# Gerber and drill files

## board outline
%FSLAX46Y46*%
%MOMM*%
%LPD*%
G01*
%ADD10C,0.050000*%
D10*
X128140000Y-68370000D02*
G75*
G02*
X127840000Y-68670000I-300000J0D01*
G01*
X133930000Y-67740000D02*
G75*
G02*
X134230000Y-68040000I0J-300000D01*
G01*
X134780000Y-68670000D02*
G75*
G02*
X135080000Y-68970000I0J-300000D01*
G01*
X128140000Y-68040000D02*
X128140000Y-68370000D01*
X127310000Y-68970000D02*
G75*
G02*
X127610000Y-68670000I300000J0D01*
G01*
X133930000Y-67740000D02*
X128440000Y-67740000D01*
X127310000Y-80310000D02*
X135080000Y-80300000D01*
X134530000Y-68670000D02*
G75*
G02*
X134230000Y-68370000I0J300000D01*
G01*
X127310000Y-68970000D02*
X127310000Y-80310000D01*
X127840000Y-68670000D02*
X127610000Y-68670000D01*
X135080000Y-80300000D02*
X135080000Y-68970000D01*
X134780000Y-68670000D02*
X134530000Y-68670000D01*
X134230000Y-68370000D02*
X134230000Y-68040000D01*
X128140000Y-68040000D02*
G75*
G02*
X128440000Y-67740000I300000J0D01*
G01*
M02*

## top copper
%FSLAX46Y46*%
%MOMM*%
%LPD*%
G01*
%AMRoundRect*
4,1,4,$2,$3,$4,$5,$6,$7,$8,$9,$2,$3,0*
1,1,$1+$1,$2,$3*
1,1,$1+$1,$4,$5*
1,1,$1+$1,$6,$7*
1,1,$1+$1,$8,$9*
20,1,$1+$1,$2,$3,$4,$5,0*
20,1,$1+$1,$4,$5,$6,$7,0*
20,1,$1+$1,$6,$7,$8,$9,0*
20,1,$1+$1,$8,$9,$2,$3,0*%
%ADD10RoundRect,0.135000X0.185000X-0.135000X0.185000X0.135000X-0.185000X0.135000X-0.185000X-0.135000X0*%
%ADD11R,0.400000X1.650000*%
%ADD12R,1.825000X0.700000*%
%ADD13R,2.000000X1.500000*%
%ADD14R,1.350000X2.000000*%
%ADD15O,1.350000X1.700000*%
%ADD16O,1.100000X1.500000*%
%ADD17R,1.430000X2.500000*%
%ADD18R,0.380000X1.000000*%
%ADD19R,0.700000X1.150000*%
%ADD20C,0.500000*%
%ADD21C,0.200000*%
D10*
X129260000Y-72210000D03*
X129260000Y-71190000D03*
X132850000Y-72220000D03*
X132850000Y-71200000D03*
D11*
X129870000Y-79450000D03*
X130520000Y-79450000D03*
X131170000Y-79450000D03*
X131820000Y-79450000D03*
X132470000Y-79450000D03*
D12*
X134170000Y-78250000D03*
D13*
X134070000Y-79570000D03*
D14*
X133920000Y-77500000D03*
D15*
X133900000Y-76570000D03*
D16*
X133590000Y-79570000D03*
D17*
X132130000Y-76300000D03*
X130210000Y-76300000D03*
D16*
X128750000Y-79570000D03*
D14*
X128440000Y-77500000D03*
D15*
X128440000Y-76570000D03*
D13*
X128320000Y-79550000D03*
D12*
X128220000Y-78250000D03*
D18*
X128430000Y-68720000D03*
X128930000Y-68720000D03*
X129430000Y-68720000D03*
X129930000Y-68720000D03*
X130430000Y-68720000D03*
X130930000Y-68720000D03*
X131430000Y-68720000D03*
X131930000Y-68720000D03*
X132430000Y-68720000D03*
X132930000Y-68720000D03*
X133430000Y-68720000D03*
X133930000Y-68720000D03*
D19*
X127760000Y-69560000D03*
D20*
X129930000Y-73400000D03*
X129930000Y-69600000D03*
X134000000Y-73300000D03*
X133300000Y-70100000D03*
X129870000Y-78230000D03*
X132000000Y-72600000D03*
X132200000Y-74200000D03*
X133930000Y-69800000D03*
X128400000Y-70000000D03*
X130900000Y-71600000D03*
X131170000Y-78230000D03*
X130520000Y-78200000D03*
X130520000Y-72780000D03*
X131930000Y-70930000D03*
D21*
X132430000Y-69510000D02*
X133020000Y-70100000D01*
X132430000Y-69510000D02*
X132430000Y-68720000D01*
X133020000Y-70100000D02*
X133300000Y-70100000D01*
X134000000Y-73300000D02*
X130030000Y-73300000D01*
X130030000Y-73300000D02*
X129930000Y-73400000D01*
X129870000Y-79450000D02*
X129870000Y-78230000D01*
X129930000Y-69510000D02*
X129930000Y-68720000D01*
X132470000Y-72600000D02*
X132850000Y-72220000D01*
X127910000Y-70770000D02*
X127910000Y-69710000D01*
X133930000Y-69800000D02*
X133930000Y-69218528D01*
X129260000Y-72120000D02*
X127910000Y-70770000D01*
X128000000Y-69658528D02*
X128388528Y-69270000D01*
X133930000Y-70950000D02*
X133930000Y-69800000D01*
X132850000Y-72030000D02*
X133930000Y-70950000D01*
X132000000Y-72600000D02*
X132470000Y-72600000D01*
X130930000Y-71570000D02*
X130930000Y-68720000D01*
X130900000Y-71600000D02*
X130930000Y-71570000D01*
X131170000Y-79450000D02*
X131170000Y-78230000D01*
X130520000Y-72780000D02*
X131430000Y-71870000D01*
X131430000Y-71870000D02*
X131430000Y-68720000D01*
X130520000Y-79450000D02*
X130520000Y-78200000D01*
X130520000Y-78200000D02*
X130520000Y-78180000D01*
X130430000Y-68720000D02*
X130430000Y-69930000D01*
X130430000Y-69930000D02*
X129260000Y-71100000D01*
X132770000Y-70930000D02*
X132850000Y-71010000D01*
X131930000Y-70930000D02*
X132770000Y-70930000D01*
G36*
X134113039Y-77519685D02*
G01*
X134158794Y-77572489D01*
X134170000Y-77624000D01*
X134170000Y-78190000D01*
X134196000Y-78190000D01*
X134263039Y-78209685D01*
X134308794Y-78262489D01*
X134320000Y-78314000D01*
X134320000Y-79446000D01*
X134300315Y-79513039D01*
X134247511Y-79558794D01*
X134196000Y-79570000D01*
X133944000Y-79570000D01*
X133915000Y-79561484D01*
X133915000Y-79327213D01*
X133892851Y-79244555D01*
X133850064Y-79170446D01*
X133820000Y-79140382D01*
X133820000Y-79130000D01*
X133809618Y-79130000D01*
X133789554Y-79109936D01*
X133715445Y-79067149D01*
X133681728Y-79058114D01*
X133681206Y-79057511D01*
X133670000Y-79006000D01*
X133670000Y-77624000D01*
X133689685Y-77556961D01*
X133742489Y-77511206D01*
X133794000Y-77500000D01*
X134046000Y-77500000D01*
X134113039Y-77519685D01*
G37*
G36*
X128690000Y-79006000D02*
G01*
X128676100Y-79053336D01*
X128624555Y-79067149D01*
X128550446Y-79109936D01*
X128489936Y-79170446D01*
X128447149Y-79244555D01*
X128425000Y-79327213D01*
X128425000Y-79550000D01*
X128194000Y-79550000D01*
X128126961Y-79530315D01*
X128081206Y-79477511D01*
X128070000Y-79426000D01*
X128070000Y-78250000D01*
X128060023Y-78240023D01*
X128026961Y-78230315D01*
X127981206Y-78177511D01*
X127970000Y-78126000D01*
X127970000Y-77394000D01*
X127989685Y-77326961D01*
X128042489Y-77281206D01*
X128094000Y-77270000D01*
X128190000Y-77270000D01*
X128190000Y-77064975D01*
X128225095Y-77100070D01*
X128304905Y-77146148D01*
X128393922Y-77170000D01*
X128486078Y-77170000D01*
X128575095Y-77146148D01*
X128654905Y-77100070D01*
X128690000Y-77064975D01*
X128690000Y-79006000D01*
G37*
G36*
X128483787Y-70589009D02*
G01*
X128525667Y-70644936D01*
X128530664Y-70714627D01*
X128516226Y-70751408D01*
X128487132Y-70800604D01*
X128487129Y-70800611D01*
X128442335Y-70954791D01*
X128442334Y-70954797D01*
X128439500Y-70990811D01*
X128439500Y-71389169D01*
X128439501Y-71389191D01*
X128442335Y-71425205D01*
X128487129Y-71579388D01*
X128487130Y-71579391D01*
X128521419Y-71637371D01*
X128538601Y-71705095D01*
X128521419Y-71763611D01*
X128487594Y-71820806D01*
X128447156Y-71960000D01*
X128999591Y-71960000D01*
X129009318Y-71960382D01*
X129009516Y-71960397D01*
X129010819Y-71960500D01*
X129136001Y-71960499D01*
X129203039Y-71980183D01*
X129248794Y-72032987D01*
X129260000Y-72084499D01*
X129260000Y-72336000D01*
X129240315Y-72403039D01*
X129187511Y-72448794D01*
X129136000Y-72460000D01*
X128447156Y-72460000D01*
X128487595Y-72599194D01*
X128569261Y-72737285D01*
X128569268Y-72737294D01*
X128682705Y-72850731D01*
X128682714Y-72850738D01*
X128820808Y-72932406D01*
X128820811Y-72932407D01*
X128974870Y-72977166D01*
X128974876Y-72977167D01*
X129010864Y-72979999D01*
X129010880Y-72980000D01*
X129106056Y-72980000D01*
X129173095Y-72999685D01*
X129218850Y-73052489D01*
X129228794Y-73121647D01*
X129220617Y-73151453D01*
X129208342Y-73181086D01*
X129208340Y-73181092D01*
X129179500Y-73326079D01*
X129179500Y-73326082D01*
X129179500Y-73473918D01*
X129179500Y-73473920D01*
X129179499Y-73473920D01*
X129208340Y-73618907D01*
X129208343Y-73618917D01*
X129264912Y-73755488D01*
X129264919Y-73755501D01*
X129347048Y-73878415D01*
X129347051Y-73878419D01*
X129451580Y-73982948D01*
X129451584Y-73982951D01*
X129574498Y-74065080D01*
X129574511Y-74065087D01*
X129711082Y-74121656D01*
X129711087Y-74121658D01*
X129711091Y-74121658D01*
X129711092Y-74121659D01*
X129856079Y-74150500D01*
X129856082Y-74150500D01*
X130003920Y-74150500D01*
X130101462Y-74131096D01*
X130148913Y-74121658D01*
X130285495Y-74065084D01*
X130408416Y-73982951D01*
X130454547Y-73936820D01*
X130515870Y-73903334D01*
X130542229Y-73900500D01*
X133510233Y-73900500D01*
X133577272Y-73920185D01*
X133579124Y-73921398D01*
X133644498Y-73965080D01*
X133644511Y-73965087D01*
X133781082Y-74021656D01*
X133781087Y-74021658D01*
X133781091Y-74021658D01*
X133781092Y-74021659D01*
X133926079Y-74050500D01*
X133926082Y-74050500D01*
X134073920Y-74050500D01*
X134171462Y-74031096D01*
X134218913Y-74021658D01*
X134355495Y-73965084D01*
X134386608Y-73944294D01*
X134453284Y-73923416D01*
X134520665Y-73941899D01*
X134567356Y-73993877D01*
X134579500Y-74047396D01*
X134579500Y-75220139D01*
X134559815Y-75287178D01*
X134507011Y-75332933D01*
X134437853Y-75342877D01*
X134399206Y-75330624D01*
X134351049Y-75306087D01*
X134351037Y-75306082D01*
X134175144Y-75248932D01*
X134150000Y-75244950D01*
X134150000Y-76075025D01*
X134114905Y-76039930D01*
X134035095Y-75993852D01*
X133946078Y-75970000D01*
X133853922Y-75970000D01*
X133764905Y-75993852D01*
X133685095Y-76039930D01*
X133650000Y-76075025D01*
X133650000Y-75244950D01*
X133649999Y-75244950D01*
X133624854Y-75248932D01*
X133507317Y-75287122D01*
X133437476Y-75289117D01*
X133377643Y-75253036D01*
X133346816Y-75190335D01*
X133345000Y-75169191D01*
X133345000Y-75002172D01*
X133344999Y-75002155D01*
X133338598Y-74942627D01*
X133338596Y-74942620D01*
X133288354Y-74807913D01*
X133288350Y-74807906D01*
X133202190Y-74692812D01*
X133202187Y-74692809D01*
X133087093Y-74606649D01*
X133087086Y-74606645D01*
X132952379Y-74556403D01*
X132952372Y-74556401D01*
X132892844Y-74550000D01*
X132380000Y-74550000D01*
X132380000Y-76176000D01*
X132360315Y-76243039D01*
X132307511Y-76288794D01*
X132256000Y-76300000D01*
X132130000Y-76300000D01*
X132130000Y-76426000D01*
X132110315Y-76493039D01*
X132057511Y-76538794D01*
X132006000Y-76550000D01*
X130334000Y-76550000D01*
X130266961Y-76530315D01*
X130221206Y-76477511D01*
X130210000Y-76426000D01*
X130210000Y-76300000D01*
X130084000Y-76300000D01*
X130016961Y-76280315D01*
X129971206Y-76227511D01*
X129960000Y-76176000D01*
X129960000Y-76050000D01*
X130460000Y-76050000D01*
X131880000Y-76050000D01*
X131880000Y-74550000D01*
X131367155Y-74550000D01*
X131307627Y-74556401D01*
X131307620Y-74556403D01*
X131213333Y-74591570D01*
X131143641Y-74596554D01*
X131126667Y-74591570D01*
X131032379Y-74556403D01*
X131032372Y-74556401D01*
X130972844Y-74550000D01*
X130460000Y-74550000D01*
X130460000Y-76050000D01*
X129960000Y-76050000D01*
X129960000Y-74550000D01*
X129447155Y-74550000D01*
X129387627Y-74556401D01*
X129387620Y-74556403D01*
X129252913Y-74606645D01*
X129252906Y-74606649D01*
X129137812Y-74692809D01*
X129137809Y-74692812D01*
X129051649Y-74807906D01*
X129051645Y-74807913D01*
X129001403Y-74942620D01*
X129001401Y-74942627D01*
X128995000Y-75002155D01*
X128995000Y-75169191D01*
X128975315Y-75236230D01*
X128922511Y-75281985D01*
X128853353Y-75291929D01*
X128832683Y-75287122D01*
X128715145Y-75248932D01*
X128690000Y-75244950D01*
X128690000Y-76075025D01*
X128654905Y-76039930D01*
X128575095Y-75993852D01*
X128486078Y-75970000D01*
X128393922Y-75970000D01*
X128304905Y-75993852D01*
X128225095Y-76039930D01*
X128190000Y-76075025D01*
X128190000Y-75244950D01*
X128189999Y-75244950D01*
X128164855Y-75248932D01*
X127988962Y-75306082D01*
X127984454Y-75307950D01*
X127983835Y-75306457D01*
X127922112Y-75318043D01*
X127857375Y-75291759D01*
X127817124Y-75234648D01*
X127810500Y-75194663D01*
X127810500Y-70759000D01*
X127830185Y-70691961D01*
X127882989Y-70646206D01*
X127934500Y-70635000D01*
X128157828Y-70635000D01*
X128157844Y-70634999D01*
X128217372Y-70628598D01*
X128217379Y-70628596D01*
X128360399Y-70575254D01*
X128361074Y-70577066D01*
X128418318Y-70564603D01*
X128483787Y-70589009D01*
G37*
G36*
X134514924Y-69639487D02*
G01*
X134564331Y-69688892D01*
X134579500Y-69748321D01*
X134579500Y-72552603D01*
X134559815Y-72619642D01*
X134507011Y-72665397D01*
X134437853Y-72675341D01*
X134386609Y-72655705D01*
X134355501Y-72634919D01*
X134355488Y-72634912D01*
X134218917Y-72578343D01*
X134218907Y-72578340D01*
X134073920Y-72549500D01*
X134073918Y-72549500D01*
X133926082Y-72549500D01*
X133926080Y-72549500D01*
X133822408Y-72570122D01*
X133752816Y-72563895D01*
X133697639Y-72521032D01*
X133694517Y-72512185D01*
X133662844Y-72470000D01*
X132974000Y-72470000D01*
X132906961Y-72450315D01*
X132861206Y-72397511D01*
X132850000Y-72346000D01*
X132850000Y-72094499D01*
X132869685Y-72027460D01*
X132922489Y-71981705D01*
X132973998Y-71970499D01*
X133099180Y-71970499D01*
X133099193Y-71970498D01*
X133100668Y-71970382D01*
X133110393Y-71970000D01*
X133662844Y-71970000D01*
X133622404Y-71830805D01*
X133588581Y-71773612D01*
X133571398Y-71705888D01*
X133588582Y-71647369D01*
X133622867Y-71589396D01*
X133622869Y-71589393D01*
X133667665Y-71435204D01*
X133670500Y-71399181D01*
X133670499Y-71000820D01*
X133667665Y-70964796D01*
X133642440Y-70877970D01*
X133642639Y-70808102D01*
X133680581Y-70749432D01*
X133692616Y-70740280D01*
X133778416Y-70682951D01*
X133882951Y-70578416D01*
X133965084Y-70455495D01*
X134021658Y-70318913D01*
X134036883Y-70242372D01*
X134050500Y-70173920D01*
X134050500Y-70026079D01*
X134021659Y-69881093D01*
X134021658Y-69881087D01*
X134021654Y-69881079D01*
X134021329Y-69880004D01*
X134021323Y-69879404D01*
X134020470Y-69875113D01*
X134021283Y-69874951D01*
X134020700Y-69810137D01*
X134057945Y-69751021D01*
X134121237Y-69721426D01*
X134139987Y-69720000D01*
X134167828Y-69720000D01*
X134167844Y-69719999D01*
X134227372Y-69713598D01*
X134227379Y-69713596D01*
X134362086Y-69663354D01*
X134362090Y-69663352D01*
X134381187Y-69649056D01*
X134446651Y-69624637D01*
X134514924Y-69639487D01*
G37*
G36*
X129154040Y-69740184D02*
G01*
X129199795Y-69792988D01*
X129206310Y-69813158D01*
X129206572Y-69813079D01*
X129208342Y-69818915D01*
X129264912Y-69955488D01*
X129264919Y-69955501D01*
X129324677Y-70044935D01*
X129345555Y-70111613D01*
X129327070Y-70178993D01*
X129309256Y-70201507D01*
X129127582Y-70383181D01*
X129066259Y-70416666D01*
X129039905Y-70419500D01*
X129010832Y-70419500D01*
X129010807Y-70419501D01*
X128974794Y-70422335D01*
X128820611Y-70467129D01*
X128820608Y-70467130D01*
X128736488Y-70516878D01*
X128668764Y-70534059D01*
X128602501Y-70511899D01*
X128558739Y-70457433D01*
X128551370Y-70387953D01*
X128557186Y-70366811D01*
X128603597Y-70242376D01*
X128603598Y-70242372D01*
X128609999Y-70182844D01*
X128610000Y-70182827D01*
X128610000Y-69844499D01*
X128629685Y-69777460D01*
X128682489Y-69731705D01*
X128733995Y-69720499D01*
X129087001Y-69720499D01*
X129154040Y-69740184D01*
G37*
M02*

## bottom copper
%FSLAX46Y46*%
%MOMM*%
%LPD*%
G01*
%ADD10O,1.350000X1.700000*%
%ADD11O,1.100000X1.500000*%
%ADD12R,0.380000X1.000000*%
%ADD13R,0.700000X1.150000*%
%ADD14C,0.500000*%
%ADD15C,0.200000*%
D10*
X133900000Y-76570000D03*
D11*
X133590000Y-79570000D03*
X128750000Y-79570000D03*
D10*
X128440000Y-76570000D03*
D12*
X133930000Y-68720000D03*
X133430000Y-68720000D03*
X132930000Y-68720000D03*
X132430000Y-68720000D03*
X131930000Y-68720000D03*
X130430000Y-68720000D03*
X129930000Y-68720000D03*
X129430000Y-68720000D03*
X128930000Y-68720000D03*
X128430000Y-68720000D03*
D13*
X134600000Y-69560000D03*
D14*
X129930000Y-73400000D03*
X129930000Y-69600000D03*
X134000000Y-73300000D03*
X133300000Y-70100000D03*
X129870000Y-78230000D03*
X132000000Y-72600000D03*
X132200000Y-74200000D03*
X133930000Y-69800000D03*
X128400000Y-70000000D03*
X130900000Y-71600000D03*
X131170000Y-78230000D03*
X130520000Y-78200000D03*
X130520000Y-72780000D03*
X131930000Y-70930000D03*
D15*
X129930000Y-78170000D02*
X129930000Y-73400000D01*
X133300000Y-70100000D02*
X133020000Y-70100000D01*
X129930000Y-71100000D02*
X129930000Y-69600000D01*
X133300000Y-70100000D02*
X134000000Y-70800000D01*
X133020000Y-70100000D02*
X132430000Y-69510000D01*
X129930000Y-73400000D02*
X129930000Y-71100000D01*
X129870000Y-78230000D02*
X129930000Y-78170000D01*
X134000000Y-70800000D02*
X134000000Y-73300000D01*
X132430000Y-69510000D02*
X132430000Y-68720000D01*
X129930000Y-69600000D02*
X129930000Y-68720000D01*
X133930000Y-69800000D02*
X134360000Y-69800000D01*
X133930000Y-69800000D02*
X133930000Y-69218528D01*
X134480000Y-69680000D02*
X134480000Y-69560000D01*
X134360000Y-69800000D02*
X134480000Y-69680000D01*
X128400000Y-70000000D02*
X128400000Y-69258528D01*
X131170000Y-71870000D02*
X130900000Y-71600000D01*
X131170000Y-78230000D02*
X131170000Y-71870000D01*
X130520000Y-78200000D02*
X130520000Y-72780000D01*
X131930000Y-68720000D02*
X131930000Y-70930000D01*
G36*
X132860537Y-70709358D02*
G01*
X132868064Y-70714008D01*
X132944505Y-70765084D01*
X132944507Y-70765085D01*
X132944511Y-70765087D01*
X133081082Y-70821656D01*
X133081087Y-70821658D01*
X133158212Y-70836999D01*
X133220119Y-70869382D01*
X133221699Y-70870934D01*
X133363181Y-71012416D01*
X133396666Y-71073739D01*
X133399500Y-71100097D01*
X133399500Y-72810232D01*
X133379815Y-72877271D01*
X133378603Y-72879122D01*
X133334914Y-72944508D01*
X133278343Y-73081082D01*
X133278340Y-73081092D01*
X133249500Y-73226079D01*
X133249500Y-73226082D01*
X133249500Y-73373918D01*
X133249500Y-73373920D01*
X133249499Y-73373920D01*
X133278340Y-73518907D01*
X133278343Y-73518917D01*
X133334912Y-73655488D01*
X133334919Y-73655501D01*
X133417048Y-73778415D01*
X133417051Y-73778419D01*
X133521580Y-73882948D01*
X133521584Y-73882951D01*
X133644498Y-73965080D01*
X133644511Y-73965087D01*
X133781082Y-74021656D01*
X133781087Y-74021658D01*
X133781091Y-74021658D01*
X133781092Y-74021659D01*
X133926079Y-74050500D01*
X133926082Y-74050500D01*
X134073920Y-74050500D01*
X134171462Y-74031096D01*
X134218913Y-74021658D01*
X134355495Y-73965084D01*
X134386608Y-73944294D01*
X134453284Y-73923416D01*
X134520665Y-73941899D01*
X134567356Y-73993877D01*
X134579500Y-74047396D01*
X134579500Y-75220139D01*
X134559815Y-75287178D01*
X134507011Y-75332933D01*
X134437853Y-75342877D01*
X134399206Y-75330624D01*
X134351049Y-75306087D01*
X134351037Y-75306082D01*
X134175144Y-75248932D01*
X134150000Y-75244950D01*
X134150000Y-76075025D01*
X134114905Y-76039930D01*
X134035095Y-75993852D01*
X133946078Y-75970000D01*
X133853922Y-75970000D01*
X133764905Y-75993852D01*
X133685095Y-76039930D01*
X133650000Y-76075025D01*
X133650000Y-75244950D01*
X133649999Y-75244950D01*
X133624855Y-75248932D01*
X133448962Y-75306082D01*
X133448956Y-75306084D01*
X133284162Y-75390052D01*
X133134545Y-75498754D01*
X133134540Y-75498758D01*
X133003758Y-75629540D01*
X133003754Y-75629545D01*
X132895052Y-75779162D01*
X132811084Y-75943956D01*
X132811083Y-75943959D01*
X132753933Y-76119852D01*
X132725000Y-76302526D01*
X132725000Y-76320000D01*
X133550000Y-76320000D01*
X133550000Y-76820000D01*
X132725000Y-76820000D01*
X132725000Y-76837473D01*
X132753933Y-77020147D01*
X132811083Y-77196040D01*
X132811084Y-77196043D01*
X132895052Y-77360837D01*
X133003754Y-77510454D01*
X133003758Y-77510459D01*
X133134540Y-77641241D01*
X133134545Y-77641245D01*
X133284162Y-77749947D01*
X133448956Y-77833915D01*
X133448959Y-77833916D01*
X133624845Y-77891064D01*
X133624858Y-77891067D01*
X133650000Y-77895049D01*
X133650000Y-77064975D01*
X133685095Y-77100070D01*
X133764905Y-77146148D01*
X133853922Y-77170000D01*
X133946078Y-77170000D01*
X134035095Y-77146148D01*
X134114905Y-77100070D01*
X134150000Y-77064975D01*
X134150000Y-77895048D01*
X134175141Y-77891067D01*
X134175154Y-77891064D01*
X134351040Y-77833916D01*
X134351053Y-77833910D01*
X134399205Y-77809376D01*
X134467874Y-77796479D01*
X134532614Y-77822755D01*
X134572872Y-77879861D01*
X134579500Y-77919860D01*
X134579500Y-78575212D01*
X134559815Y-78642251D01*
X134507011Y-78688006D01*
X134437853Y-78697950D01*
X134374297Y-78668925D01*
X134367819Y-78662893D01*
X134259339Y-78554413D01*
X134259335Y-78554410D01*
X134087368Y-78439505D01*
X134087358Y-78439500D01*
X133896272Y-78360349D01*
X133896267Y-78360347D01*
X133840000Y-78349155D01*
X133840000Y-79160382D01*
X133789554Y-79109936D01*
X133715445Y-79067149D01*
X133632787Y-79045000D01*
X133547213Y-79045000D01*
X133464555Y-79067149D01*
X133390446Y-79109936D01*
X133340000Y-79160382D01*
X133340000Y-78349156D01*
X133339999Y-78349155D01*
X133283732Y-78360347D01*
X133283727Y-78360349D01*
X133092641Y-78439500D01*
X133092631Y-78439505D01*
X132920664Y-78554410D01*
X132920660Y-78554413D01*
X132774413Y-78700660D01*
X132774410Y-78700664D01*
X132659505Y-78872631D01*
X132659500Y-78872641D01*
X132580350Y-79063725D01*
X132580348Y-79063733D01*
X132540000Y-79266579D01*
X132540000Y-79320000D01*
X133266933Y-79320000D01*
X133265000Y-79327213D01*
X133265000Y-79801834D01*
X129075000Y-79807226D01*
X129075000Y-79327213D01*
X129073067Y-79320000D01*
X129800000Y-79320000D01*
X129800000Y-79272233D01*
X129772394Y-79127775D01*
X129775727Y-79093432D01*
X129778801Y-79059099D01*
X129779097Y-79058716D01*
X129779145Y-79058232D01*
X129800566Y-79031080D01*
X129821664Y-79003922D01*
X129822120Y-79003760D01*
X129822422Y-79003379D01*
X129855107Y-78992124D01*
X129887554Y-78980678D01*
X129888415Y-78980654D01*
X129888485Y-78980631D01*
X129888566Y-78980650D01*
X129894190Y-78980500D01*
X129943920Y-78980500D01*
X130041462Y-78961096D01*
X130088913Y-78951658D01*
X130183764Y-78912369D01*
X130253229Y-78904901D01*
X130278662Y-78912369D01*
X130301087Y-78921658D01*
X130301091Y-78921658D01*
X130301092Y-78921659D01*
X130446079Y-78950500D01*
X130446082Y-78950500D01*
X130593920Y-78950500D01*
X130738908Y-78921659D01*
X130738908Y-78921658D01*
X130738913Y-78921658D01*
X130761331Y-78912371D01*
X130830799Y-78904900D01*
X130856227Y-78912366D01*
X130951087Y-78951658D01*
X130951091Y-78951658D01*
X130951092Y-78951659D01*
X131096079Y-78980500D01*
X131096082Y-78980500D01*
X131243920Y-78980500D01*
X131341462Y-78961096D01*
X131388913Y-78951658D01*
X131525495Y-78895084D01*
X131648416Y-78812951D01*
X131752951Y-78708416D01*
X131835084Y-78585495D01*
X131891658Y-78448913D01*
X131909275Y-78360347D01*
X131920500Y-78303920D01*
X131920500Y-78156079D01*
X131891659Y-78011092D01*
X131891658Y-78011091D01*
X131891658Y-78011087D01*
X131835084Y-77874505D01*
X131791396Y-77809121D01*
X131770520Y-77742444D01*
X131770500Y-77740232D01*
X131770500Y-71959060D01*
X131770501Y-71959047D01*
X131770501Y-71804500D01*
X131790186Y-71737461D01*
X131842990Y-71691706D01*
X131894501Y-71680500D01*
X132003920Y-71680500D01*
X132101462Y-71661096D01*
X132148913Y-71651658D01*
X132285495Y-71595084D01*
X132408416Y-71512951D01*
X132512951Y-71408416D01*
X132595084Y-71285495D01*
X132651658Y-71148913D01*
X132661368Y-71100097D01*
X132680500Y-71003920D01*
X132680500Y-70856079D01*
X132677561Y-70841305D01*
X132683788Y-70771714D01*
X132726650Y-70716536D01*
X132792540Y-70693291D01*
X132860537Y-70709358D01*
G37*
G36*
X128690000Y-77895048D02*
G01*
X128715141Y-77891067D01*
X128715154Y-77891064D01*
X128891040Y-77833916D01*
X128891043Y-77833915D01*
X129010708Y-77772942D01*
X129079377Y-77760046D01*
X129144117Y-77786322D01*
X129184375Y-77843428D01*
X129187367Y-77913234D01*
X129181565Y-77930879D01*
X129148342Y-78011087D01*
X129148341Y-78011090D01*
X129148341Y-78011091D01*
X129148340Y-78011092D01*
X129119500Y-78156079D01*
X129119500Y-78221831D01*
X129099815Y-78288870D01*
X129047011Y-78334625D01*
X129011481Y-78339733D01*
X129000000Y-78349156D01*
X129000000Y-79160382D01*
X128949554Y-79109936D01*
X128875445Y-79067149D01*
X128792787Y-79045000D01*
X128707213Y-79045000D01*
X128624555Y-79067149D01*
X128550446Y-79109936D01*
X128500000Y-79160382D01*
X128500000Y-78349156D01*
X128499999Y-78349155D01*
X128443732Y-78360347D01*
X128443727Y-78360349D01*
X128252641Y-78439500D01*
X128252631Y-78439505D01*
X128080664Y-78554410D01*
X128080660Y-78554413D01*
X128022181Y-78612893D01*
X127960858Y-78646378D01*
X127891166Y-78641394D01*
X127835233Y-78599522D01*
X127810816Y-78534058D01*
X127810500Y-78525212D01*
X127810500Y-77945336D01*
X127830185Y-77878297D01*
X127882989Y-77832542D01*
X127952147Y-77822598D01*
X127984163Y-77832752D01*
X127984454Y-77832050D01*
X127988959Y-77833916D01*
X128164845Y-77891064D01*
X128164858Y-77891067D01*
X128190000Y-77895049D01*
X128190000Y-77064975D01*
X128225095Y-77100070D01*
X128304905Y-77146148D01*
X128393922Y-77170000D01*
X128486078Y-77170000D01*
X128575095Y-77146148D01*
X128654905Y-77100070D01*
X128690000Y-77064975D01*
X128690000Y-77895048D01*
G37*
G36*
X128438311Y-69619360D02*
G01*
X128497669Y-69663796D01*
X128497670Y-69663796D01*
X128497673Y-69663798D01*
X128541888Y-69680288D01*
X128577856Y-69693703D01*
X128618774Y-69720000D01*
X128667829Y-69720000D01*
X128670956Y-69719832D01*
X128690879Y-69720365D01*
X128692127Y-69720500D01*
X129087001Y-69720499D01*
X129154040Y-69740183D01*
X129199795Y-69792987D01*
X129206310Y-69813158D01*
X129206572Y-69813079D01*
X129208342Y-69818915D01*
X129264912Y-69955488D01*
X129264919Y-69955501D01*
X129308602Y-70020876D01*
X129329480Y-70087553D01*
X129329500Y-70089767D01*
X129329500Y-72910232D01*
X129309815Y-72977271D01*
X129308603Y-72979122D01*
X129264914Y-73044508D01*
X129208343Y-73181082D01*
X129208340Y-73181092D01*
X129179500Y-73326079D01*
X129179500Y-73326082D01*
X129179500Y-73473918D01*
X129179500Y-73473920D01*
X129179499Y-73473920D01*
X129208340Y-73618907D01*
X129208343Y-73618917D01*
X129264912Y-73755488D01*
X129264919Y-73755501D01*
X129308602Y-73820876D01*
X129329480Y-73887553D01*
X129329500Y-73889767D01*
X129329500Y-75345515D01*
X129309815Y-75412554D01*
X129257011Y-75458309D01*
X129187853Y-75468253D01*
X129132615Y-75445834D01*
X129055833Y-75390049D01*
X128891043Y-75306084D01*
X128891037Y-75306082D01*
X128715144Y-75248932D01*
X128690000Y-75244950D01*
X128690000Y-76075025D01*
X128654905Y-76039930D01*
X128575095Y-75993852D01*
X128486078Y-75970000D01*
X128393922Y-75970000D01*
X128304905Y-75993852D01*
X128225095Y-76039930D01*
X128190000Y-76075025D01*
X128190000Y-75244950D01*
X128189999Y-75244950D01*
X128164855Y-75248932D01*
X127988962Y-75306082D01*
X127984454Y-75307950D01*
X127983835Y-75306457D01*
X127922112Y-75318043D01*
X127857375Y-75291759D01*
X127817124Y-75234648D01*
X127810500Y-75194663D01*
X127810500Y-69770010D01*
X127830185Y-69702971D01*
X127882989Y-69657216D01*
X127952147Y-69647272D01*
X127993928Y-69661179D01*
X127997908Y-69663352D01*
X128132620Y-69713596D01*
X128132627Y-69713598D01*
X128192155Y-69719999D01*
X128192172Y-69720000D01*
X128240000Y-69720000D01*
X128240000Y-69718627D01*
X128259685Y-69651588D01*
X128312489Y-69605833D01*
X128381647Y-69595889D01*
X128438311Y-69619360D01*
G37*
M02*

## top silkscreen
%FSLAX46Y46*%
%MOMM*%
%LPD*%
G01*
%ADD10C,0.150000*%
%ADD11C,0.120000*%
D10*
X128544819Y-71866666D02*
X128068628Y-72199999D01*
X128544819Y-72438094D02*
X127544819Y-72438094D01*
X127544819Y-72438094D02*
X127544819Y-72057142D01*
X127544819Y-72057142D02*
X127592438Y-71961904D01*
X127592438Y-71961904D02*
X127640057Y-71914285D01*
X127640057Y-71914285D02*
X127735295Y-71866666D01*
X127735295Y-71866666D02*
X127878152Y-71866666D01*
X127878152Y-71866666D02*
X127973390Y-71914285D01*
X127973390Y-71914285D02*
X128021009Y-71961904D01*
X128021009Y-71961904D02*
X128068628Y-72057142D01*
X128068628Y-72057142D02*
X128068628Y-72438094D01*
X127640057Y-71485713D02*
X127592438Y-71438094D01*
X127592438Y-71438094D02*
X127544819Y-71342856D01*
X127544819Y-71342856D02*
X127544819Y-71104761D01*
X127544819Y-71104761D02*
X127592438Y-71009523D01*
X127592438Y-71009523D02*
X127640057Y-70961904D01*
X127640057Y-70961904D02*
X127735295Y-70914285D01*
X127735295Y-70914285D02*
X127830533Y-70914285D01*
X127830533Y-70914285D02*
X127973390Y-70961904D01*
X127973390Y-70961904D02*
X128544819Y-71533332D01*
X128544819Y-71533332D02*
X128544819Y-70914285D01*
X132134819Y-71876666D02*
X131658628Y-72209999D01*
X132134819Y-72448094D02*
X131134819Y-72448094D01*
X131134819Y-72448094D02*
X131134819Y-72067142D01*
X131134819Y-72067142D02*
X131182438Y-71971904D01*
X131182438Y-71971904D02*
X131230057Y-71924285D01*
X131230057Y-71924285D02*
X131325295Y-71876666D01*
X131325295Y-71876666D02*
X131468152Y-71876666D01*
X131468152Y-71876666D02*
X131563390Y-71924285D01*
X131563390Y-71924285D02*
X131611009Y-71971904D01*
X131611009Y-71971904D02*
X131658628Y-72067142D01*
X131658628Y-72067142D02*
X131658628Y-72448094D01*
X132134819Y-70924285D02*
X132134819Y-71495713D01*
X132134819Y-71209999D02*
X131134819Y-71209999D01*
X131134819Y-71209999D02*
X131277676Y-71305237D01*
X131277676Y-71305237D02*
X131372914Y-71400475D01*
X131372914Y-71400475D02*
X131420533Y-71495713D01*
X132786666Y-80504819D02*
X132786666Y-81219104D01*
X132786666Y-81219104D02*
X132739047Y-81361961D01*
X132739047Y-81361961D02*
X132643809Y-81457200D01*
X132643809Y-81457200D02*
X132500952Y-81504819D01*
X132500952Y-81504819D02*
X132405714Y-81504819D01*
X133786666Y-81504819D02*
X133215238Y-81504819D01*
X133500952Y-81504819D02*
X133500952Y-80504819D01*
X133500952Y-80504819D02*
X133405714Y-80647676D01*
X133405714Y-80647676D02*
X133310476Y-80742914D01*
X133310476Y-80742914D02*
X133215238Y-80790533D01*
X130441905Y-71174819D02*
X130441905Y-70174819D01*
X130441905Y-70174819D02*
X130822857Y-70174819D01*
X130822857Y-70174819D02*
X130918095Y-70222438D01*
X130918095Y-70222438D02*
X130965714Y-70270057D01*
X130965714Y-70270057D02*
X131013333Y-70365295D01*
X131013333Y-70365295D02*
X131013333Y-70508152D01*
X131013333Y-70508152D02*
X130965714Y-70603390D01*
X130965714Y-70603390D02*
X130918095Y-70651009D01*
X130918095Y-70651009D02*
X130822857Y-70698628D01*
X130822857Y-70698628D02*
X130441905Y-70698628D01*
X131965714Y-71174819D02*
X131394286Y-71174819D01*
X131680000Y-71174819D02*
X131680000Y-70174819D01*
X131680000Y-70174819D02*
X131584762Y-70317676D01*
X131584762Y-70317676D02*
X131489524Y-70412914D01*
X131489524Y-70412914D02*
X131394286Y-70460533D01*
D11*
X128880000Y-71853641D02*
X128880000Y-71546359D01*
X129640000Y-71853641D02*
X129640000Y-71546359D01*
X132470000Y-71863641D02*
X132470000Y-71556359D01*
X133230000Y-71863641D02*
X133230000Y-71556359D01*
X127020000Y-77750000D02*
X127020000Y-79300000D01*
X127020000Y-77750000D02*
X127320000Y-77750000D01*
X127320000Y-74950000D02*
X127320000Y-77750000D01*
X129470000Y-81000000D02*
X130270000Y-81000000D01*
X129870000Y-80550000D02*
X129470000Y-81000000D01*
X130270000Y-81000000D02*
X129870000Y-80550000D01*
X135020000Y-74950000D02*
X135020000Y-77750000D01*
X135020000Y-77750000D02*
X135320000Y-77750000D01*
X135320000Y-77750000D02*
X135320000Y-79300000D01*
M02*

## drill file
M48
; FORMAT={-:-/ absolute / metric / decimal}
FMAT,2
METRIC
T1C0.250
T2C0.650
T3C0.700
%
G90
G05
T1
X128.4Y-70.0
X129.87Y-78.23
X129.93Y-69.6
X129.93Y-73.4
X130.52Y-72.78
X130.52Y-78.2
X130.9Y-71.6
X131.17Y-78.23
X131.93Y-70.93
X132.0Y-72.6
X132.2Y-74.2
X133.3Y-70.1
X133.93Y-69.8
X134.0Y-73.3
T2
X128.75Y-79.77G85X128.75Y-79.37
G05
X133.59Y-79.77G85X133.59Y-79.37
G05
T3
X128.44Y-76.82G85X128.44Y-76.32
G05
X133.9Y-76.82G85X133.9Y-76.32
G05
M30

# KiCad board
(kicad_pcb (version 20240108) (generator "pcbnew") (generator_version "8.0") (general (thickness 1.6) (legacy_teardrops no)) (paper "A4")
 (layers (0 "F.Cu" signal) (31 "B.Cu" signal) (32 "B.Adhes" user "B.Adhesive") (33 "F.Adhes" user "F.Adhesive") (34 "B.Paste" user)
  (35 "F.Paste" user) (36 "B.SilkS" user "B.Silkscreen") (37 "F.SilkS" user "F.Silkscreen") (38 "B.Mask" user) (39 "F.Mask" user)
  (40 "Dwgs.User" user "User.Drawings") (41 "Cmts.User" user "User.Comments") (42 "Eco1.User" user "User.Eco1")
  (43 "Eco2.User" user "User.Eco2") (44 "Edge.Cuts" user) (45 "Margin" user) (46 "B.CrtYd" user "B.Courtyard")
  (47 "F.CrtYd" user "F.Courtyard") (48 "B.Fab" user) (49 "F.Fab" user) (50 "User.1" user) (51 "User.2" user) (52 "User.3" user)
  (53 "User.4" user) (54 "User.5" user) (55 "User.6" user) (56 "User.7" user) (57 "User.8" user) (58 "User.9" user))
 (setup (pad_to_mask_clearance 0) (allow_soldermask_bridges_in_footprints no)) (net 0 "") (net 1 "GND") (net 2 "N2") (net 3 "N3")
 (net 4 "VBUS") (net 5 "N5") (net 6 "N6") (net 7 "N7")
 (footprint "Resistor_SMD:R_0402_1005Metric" (layer "F.Cu") (at 129.26 71.7 90)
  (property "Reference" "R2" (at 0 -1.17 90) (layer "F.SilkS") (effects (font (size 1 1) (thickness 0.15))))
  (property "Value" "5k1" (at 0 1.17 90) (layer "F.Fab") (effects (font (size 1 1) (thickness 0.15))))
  (fp_line (start -0.153641 -0.38) (end 0.153641 -0.38) (stroke (width 0.12) (type solid)) (layer "F.SilkS"))
  (fp_line (start -0.153641 0.38) (end 0.153641 0.38) (stroke (width 0.12) (type solid)) (layer "F.SilkS"))
  (pad "1" smd roundrect (at -0.51 0 90) (size 0.54 0.64) (layers "F.Cu" "F.Paste" "F.Mask") (roundrect_rratio 0.25) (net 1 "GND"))
  (pad "2" smd roundrect (at 0.51 0 90) (size 0.54 0.64) (layers "F.Cu" "F.Paste" "F.Mask") (roundrect_rratio 0.25) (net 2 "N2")))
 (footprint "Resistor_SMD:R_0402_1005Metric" (layer "F.Cu") (at 132.85 71.71 90)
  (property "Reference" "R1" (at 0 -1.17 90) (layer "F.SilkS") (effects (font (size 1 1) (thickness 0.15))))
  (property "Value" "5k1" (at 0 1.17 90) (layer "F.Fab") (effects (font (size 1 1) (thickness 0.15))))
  (fp_line (start -0.153641 -0.38) (end 0.153641 -0.38) (stroke (width 0.12) (type solid)) (layer "F.SilkS"))
  (fp_line (start -0.153641 0.38) (end 0.153641 0.38) (stroke (width 0.12) (type solid)) (layer "F.SilkS"))
  (pad "1" smd roundrect (at -0.51 0 90) (size 0.54 0.64) (layers "F.Cu" "F.Paste" "F.Mask") (roundrect_rratio 0.25) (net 1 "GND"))
  (pad "2" smd roundrect (at 0.51 0 90) (size 0.54 0.64) (layers "F.Cu" "F.Paste" "F.Mask") (roundrect_rratio 0.25) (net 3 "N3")))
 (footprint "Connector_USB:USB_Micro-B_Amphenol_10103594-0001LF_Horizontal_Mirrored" (layer "F.Cu") (at 130.655 77.685 180)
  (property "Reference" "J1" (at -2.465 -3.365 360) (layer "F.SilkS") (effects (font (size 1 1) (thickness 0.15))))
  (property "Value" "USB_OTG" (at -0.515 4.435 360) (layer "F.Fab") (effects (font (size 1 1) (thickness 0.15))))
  (fp_line (start 3.635 -0.065) (end 3.635 -1.615) (stroke (width 0.12) (type solid)) (layer "F.SilkS"))
  (fp_line (start 3.635 -0.065) (end 3.335 -0.065) (stroke (width 0.12) (type solid)) (layer "F.SilkS"))
  (fp_line (start 3.335 2.735) (end 3.335 -0.065) (stroke (width 0.12) (type solid)) (layer "F.SilkS"))
  (fp_line (start 1.185 -3.315) (end 0.385 -3.315) (stroke (width 0.12) (type solid)) (layer "F.SilkS"))
  (fp_line (start 0.785 -2.865) (end 1.185 -3.315) (stroke (width 0.12) (type solid)) (layer "F.SilkS"))
  (fp_line (start 0.385 -3.315) (end 0.785 -2.865) (stroke (width 0.12) (type solid)) (layer "F.SilkS"))
  (fp_line (start -4.365 2.735) (end -4.365 -0.065) (stroke (width 0.12) (type solid)) (layer "F.SilkS"))
  (fp_line (start -4.365 -0.065) (end -4.665 -0.065) (stroke (width 0.12) (type solid)) (layer "F.SilkS"))
  (fp_line (start -4.665 -0.065) (end -4.665 -1.615) (stroke (width 0.12) (type solid)) (layer "F.SilkS"))
  (pad "1" smd rect (at 0.785 -1.765 90) (size 1.65 0.4) (layers "F.Cu" "F.Paste" "F.Mask") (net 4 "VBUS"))
  (pad "2" smd rect (at 0.135 -1.765 90) (size 1.65 0.4) (layers "F.Cu" "F.Paste" "F.Mask") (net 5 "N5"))
  (pad "3" smd rect (at -0.515 -1.765 90) (size 1.65 0.4) (layers "F.Cu" "F.Paste" "F.Mask") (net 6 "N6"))
  (pad "4" smd rect (at -1.165 -1.765 90) (size 1.65 0.4) (layers "F.Cu" "F.Paste" "F.Mask") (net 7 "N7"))
  (pad "5" smd rect (at -1.815 -1.765 90) (size 1.65 0.4) (layers "F.Cu" "F.Paste" "F.Mask") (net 1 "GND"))
  (pad "6" smd rect (at -3.515 -0.565 180) (size 1.825 0.7) (layers "F.Cu" "F.Paste" "F.Mask") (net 1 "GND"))
  (pad "6" smd rect (at -3.415 -1.885 180) (size 2 1.5) (layers "F.Cu" "F.Paste" "F.Mask") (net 1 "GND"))
  (pad "6" smd rect (at -3.265 0.185 180) (size 1.35 2) (layers "F.Cu" "F.Paste" "F.Mask") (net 1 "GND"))
  (pad "6" thru_hole oval (at -3.245 1.115 90) (size 1.7 1.35) (drill oval 1.2 0.7) (layers "*.Cu" "*.Mask") (remove_unused_layers no)
   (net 1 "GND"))
  (pad "6" thru_hole oval (at -2.935 -1.885 90) (size 1.5 1.1) (drill oval 1.05 0.65) (layers "*.Cu" "*.Mask") (remove_unused_layers no)
   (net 1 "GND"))
  (pad "6" smd rect (at -1.475 1.385 90) (size 2.5 1.43) (layers "F.Cu" "F.Paste" "F.Mask") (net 1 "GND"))
  (pad "6" smd rect (at 0.445 1.385 90) (size 2.5 1.43) (layers "F.Cu" "F.Paste" "F.Mask") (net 1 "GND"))
  (pad "6" thru_hole oval (at 1.905 -1.885 90) (size 1.5 1.1) (drill oval 1.05 0.65) (layers "*.Cu" "*.Mask") (remove_unused_layers no)
   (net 1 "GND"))
  (pad "6" smd rect (at 2.215 0.185 180) (size 1.35 2) (layers "F.Cu" "F.Paste" "F.Mask") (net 1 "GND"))
  (pad "6" thru_hole oval (at 2.215 1.115 90) (size 1.7 1.35) (drill oval 1.2 0.7) (layers "*.Cu" "*.Mask") (remove_unused_layers no)
   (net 1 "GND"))
  (pad "6" smd rect (at 2.335 -1.865 180) (size 2 1.5) (layers "F.Cu" "F.Paste" "F.Mask") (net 1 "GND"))
  (pad "6" smd rect (at 2.435 -0.565 180) (size 1.825 0.7) (layers "F.Cu" "F.Paste" "F.Mask") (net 1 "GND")))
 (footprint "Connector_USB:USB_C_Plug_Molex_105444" (layer "F.Cu") (at 131.18 68.68)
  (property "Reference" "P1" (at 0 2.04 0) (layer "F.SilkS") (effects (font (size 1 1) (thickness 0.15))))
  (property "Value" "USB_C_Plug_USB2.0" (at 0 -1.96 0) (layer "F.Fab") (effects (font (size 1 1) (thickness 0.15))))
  (pad "A1" smd rect (at -2.75 0.04) (size 0.38 1) (layers "F.Cu" "F.Paste" "F.Mask") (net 1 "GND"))
  (pad "A2" smd rect (at -2.25 0.04) (size 0.38 1) (layers "F.Cu" "F.Paste" "F.Mask"))
  (pad "A3" smd rect (at -1.75 0.04) (size 0.38 1) (layers "F.Cu" "F.Paste" "F.Mask"))
  (pad "A4" smd rect (at -1.25 0.04) (size 0.38 1) (layers "F.Cu" "F.Paste" "F.Mask") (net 4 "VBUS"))
  (pad "A5" smd rect (at -0.75 0.04) (size 0.38 1) (layers "F.Cu" "F.Paste" "F.Mask") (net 2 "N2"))
  (pad "A6" smd rect (at -0.25 0.04) (size 0.38 1) (layers "F.Cu" "F.Paste" "F.Mask") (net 6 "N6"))
  (pad "A7" smd rect (at 0.25 0.04) (size 0.38 1) (layers "F.Cu" "F.Paste" "F.Mask") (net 5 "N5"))
  (pad "A8" smd rect (at 0.75 0.04) (size 0.38 1) (layers "F.Cu" "F.Paste" "F.Mask"))
  (pad "A9" smd rect (at 1.25 0.04) (size 0.38 1) (layers "F.Cu" "F.Paste" "F.Mask") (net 4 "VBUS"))
  (pad "A10" smd rect (at 1.75 0.04) (size 0.38 1) (layers "F.Cu" "F.Paste" "F.Mask"))
  (pad "A11" smd rect (at 2.25 0.04) (size 0.38 1) (layers "F.Cu" "F.Paste" "F.Mask"))
  (pad "A12" smd rect (at 2.75 0.04) (size 0.38 1) (layers "F.Cu" "F.Paste" "F.Mask") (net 1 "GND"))
  (pad "B1" smd rect (at 2.75 0.04) (size 0.38 1) (layers "B.Cu" "B.Paste" "B.Mask") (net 1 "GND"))
  (pad "B2" smd rect (at 2.25 0.04) (size 0.38 1) (layers "B.Cu" "B.Paste" "B.Mask"))
  (pad "B3" smd rect (at 1.75 0.04) (size 0.38 1) (layers "B.Cu" "B.Paste" "B.Mask"))
  (pad "B4" smd rect (at 1.25 0.04) (size 0.38 1) (layers "B.Cu" "B.Paste" "B.Mask") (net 4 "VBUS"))
  (pad "B5" smd rect (at 0.75 0.04) (size 0.38 1) (layers "B.Cu" "B.Paste" "B.Mask") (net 3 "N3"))
  (pad "B8" smd rect (at -0.75 0.04) (size 0.38 1) (layers "B.Cu" "B.Paste" "B.Mask"))
  (pad "B9" smd rect (at -1.25 0.04) (size 0.38 1) (layers "B.Cu" "B.Paste" "B.Mask") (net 4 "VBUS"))
  (pad "B10" smd rect (at -1.75 0.04) (size 0.38 1) (layers "B.Cu" "B.Paste" "B.Mask"))
  (pad "B11" smd rect (at -2.25 0.04) (size 0.38 1) (layers "B.Cu" "B.Paste" "B.Mask"))
  (pad "B12" smd rect (at -2.75 0.04) (size 0.38 1) (layers "B.Cu" "B.Paste" "B.Mask") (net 1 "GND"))
  (pad "S1" smd rect (at -3.42 0.88) (size 0.7 1.15) (layers "F.Cu" "F.Paste" "F.Mask") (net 1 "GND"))
  (pad "S1" smd rect (at 3.42 0.88) (size 0.7 1.15) (layers "B.Cu" "B.Paste" "B.Mask") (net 1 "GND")))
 (gr_arc (start 128.14 68.37) (mid 128.052132 68.582132) (end 127.84 68.67) (stroke (width 0.05) (type default)) (layer "Edge.Cuts"))
 (gr_arc (start 133.93 67.74) (mid 134.142132 67.827868) (end 134.23 68.04) (stroke (width 0.05) (type default)) (layer "Edge.Cuts"))
 (gr_arc (start 134.78 68.67) (mid 134.992132 68.757868) (end 135.08 68.97) (stroke (width 0.05) (type default)) (layer "Edge.Cuts"))
 (gr_line (start 128.14 68.04) (end 128.14 68.37) (stroke (width 0.05) (type default)) (layer "Edge.Cuts"))
 (gr_arc (start 127.31 68.97) (mid 127.397868 68.757868) (end 127.61 68.67) (stroke (width 0.05) (type default)) (layer "Edge.Cuts"))
 (gr_line (start 133.93 67.74) (end 128.44 67.74) (stroke (width 0.05) (type default)) (layer "Edge.Cuts"))
 (gr_line (start 127.31 80.31) (end 135.08 80.3) (stroke (width 0.05) (type default)) (layer "Edge.Cuts"))
 (gr_arc (start 134.53 68.67) (mid 134.317868 68.582132) (end 134.23 68.37) (stroke (width 0.05) (type default)) (layer "Edge.Cuts"))
 (gr_line (start 127.31 68.97) (end 127.31 80.31) (stroke (width 0.05) (type default)) (layer "Edge.Cuts"))
 (gr_line (start 127.84 68.67) (end 127.61 68.67) (stroke (width 0.05) (type default)) (layer "Edge.Cuts"))
 (gr_line (start 135.08 80.3) (end 135.08 68.97) (stroke (width 0.05) (type default)) (layer "Edge.Cuts"))
 (gr_line (start 134.78 68.67) (end 134.53 68.67) (stroke (width 0.05) (type default)) (layer "Edge.Cuts"))
 (gr_line (start 134.23 68.37) (end 134.23 68.04) (stroke (width 0.05) (type default)) (layer "Edge.Cuts"))
 (gr_arc (start 128.14 68.04) (mid 128.227868 67.827868) (end 128.44 67.74) (stroke (width 0.05) (type default)) (layer "Edge.Cuts"))
 (segment (start 132.43 69.51) (end 133.02 70.1) (width 0.2) (layer "F.Cu") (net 4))
 (segment (start 132.43 69.51) (end 132.43 68.72) (width 0.2) (layer "F.Cu") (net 4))
 (segment (start 133.02 70.1) (end 133.3 70.1) (width 0.2) (layer "F.Cu") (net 4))
 (segment (start 134 73.3) (end 130.03 73.3) (width 0.2) (layer "F.Cu") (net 4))
 (segment (start 130.03 73.3) (end 129.93 73.4) (width 0.2) (layer "F.Cu") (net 4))
 (segment (start 129.87 79.45) (end 129.87 78.23) (width 0.2) (layer "F.Cu") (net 4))
 (segment (start 129.93 69.51) (end 129.93 68.72) (width 0.2) (layer "F.Cu") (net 4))
 (via (at 129.93 73.4) (size 0.5) (drill 0.25) (layers "F.Cu" "B.Cu") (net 4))
 (via (at 129.93 69.6) (size 0.5) (drill 0.25) (layers "F.Cu" "B.Cu") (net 4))
 (via (at 134 73.3) (size 0.5) (drill 0.25) (layers "F.Cu" "B.Cu") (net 4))
 (via (at 133.3 70.1) (size 0.5) (drill 0.25) (layers "F.Cu" "B.Cu") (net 4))
 (via (at 129.87 78.23) (size 0.5) (drill 0.25) (layers "F.Cu" "B.Cu") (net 4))
 (segment (start 129.93 78.17) (end 129.93 73.4) (width 0.2) (layer "B.Cu") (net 4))
 (segment (start 133.3 70.1) (end 133.02 70.1) (width 0.2) (layer "B.Cu") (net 4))
 (segment (start 129.93 71.1) (end 129.93 69.6) (width 0.2) (layer "B.Cu") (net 4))
 (segment (start 133.3 70.1) (end 134 70.8) (width 0.2) (layer "B.Cu") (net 4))
 (segment (start 133.02 70.1) (end 132.43 69.51) (width 0.2) (layer "B.Cu") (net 4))
 (segment (start 129.93 73.4) (end 129.93 71.1) (width 0.2) (layer "B.Cu") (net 4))
 (segment (start 129.87 78.23) (end 129.93 78.17) (width 0.2) (layer "B.Cu") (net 4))
 (segment (start 134 70.8) (end 134 73.3) (width 0.2) (layer "B.Cu") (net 4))
 (segment (start 132.43 69.51) (end 132.43 68.72) (width 0.2) (layer "B.Cu") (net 4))
 (segment (start 129.93 69.6) (end 129.93 68.72) (width 0.2) (layer "B.Cu") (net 4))
 (segment (start 132.47 72.6) (end 132.85 72.22) (width 0.2) (layer "F.Cu") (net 1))
 (segment (start 127.91 70.77) (end 127.91 69.71) (width 0.2) (layer "F.Cu") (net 1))
 (segment (start 133.93 69.8) (end 133.93 69.218528) (width 0.2) (layer "F.Cu") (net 1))
 (segment (start 129.26 72.12) (end 127.91 70.77) (width 0.2) (layer "F.Cu") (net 1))
 (segment (start 128 69.658528) (end 128.388528 69.27) (width 0.2) (layer "F.Cu") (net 1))
 (segment (start 133.93 70.95) (end 133.93 69.8) (width 0.2) (layer "F.Cu") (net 1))
 (segment (start 132.85 72.03) (end 133.93 70.95) (width 0.2) (layer "F.Cu") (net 1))
 (segment (start 132 72.6) (end 132.47 72.6) (width 0.2) (layer "F.Cu") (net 1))
 (via (at 132 72.6) (size 0.5) (drill 0.25) (layers "F.Cu" "B.Cu") (free yes) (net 1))
 (via (at 132.2 74.2) (size 0.5) (drill 0.25) (layers "F.Cu" "B.Cu") (free yes) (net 1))
 (via (at 133.93 69.8) (size 0.5) (drill 0.25) (layers "F.Cu" "B.Cu") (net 1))
 (via (at 128.4 70) (size 0.5) (drill 0.25) (layers "F.Cu" "B.Cu") (free yes) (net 1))
 (segment (start 133.93 69.8) (end 134.36 69.8) (width 0.2) (layer "B.Cu") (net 1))
 (segment (start 133.93 69.8) (end 133.93 69.218528) (width 0.2) (layer "B.Cu") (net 1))
 (segment (start 134.48 69.68) (end 134.48 69.56) (width 0.2) (layer "B.Cu") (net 1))
 (segment (start 134.36 69.8) (end 134.48 69.68) (width 0.2) (layer "B.Cu") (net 1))
 (segment (start 128.4 70) (end 128.4 69.258528) (width 0.2) (layer "B.Cu") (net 1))
 (segment (start 130.93 71.57) (end 130.93 68.72) (width 0.2) (layer "F.Cu") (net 6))
 (segment (start 130.9 71.6) (end 130.93 71.57) (width 0.2) (layer "F.Cu") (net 6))
 (segment (start 131.17 79.45) (end 131.17 78.23) (width 0.2) (layer "F.Cu") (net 6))
 (via (at 130.9 71.6) (size 0.5) (drill 0.25) (layers "F.Cu" "B.Cu") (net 6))
 (via (at 131.17 78.23) (size 0.5) (drill 0.25) (layers "F.Cu" "B.Cu") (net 6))
 (segment (start 131.17 71.87) (end 130.9 71.6) (width 0.2) (layer "B.Cu") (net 6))
 (segment (start 131.17 78.23) (end 131.17 71.87) (width 0.2) (layer "B.Cu") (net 6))
 (segment (start 130.52 72.78) (end 131.43 71.87) (width 0.2) (layer "F.Cu") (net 5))
 (segment (start 131.43 71.87) (end 131.43 68.72) (width 0.2) (layer "F.Cu") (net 5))
 (segment (start 130.52 79.45) (end 130.52 78.2) (width 0.2) (layer "F.Cu") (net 5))
 (segment (start 130.52 78.2) (end 130.52 78.18) (width 0.2) (layer "F.Cu") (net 5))
 (via (at 130.52 78.2) (size 0.5) (drill 0.25) (layers "F.Cu" "B.Cu") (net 5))
 (via (at 130.52 72.78) (size 0.5) (drill 0.25) (layers "F.Cu" "B.Cu") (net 5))
 (segment (start 130.52 78.2) (end 130.52 72.78) (width 0.2) (layer "B.Cu") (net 5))
 (segment (start 130.43 68.72) (end 130.43 69.93) (width 0.2) (layer "F.Cu") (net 2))
 (segment (start 130.43 69.93) (end 129.26 71.1) (width 0.2) (layer "F.Cu") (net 2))
 (segment (start 132.77 70.93) (end 132.85 71.01) (width 0.2) (layer "F.Cu") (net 3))
 (segment (start 131.93 70.93) (end 132.77 70.93) (width 0.2) (layer "F.Cu") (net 3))
 (via (at 131.93 70.93) (size 0.5) (drill 0.25) (layers "F.Cu" "B.Cu") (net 3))
 (segment (start 131.93 68.72) (end 131.93 70.93) (width 0.2) (layer "B.Cu") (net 3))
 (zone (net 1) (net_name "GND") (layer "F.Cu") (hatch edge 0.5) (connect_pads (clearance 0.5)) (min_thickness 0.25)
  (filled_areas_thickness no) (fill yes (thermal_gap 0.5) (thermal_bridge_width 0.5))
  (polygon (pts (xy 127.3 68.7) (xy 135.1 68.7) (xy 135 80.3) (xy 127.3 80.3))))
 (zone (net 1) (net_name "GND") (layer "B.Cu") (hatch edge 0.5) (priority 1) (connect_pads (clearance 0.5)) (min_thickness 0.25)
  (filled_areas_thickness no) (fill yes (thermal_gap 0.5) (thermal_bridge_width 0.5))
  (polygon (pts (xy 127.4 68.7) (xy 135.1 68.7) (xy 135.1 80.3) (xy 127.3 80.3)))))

